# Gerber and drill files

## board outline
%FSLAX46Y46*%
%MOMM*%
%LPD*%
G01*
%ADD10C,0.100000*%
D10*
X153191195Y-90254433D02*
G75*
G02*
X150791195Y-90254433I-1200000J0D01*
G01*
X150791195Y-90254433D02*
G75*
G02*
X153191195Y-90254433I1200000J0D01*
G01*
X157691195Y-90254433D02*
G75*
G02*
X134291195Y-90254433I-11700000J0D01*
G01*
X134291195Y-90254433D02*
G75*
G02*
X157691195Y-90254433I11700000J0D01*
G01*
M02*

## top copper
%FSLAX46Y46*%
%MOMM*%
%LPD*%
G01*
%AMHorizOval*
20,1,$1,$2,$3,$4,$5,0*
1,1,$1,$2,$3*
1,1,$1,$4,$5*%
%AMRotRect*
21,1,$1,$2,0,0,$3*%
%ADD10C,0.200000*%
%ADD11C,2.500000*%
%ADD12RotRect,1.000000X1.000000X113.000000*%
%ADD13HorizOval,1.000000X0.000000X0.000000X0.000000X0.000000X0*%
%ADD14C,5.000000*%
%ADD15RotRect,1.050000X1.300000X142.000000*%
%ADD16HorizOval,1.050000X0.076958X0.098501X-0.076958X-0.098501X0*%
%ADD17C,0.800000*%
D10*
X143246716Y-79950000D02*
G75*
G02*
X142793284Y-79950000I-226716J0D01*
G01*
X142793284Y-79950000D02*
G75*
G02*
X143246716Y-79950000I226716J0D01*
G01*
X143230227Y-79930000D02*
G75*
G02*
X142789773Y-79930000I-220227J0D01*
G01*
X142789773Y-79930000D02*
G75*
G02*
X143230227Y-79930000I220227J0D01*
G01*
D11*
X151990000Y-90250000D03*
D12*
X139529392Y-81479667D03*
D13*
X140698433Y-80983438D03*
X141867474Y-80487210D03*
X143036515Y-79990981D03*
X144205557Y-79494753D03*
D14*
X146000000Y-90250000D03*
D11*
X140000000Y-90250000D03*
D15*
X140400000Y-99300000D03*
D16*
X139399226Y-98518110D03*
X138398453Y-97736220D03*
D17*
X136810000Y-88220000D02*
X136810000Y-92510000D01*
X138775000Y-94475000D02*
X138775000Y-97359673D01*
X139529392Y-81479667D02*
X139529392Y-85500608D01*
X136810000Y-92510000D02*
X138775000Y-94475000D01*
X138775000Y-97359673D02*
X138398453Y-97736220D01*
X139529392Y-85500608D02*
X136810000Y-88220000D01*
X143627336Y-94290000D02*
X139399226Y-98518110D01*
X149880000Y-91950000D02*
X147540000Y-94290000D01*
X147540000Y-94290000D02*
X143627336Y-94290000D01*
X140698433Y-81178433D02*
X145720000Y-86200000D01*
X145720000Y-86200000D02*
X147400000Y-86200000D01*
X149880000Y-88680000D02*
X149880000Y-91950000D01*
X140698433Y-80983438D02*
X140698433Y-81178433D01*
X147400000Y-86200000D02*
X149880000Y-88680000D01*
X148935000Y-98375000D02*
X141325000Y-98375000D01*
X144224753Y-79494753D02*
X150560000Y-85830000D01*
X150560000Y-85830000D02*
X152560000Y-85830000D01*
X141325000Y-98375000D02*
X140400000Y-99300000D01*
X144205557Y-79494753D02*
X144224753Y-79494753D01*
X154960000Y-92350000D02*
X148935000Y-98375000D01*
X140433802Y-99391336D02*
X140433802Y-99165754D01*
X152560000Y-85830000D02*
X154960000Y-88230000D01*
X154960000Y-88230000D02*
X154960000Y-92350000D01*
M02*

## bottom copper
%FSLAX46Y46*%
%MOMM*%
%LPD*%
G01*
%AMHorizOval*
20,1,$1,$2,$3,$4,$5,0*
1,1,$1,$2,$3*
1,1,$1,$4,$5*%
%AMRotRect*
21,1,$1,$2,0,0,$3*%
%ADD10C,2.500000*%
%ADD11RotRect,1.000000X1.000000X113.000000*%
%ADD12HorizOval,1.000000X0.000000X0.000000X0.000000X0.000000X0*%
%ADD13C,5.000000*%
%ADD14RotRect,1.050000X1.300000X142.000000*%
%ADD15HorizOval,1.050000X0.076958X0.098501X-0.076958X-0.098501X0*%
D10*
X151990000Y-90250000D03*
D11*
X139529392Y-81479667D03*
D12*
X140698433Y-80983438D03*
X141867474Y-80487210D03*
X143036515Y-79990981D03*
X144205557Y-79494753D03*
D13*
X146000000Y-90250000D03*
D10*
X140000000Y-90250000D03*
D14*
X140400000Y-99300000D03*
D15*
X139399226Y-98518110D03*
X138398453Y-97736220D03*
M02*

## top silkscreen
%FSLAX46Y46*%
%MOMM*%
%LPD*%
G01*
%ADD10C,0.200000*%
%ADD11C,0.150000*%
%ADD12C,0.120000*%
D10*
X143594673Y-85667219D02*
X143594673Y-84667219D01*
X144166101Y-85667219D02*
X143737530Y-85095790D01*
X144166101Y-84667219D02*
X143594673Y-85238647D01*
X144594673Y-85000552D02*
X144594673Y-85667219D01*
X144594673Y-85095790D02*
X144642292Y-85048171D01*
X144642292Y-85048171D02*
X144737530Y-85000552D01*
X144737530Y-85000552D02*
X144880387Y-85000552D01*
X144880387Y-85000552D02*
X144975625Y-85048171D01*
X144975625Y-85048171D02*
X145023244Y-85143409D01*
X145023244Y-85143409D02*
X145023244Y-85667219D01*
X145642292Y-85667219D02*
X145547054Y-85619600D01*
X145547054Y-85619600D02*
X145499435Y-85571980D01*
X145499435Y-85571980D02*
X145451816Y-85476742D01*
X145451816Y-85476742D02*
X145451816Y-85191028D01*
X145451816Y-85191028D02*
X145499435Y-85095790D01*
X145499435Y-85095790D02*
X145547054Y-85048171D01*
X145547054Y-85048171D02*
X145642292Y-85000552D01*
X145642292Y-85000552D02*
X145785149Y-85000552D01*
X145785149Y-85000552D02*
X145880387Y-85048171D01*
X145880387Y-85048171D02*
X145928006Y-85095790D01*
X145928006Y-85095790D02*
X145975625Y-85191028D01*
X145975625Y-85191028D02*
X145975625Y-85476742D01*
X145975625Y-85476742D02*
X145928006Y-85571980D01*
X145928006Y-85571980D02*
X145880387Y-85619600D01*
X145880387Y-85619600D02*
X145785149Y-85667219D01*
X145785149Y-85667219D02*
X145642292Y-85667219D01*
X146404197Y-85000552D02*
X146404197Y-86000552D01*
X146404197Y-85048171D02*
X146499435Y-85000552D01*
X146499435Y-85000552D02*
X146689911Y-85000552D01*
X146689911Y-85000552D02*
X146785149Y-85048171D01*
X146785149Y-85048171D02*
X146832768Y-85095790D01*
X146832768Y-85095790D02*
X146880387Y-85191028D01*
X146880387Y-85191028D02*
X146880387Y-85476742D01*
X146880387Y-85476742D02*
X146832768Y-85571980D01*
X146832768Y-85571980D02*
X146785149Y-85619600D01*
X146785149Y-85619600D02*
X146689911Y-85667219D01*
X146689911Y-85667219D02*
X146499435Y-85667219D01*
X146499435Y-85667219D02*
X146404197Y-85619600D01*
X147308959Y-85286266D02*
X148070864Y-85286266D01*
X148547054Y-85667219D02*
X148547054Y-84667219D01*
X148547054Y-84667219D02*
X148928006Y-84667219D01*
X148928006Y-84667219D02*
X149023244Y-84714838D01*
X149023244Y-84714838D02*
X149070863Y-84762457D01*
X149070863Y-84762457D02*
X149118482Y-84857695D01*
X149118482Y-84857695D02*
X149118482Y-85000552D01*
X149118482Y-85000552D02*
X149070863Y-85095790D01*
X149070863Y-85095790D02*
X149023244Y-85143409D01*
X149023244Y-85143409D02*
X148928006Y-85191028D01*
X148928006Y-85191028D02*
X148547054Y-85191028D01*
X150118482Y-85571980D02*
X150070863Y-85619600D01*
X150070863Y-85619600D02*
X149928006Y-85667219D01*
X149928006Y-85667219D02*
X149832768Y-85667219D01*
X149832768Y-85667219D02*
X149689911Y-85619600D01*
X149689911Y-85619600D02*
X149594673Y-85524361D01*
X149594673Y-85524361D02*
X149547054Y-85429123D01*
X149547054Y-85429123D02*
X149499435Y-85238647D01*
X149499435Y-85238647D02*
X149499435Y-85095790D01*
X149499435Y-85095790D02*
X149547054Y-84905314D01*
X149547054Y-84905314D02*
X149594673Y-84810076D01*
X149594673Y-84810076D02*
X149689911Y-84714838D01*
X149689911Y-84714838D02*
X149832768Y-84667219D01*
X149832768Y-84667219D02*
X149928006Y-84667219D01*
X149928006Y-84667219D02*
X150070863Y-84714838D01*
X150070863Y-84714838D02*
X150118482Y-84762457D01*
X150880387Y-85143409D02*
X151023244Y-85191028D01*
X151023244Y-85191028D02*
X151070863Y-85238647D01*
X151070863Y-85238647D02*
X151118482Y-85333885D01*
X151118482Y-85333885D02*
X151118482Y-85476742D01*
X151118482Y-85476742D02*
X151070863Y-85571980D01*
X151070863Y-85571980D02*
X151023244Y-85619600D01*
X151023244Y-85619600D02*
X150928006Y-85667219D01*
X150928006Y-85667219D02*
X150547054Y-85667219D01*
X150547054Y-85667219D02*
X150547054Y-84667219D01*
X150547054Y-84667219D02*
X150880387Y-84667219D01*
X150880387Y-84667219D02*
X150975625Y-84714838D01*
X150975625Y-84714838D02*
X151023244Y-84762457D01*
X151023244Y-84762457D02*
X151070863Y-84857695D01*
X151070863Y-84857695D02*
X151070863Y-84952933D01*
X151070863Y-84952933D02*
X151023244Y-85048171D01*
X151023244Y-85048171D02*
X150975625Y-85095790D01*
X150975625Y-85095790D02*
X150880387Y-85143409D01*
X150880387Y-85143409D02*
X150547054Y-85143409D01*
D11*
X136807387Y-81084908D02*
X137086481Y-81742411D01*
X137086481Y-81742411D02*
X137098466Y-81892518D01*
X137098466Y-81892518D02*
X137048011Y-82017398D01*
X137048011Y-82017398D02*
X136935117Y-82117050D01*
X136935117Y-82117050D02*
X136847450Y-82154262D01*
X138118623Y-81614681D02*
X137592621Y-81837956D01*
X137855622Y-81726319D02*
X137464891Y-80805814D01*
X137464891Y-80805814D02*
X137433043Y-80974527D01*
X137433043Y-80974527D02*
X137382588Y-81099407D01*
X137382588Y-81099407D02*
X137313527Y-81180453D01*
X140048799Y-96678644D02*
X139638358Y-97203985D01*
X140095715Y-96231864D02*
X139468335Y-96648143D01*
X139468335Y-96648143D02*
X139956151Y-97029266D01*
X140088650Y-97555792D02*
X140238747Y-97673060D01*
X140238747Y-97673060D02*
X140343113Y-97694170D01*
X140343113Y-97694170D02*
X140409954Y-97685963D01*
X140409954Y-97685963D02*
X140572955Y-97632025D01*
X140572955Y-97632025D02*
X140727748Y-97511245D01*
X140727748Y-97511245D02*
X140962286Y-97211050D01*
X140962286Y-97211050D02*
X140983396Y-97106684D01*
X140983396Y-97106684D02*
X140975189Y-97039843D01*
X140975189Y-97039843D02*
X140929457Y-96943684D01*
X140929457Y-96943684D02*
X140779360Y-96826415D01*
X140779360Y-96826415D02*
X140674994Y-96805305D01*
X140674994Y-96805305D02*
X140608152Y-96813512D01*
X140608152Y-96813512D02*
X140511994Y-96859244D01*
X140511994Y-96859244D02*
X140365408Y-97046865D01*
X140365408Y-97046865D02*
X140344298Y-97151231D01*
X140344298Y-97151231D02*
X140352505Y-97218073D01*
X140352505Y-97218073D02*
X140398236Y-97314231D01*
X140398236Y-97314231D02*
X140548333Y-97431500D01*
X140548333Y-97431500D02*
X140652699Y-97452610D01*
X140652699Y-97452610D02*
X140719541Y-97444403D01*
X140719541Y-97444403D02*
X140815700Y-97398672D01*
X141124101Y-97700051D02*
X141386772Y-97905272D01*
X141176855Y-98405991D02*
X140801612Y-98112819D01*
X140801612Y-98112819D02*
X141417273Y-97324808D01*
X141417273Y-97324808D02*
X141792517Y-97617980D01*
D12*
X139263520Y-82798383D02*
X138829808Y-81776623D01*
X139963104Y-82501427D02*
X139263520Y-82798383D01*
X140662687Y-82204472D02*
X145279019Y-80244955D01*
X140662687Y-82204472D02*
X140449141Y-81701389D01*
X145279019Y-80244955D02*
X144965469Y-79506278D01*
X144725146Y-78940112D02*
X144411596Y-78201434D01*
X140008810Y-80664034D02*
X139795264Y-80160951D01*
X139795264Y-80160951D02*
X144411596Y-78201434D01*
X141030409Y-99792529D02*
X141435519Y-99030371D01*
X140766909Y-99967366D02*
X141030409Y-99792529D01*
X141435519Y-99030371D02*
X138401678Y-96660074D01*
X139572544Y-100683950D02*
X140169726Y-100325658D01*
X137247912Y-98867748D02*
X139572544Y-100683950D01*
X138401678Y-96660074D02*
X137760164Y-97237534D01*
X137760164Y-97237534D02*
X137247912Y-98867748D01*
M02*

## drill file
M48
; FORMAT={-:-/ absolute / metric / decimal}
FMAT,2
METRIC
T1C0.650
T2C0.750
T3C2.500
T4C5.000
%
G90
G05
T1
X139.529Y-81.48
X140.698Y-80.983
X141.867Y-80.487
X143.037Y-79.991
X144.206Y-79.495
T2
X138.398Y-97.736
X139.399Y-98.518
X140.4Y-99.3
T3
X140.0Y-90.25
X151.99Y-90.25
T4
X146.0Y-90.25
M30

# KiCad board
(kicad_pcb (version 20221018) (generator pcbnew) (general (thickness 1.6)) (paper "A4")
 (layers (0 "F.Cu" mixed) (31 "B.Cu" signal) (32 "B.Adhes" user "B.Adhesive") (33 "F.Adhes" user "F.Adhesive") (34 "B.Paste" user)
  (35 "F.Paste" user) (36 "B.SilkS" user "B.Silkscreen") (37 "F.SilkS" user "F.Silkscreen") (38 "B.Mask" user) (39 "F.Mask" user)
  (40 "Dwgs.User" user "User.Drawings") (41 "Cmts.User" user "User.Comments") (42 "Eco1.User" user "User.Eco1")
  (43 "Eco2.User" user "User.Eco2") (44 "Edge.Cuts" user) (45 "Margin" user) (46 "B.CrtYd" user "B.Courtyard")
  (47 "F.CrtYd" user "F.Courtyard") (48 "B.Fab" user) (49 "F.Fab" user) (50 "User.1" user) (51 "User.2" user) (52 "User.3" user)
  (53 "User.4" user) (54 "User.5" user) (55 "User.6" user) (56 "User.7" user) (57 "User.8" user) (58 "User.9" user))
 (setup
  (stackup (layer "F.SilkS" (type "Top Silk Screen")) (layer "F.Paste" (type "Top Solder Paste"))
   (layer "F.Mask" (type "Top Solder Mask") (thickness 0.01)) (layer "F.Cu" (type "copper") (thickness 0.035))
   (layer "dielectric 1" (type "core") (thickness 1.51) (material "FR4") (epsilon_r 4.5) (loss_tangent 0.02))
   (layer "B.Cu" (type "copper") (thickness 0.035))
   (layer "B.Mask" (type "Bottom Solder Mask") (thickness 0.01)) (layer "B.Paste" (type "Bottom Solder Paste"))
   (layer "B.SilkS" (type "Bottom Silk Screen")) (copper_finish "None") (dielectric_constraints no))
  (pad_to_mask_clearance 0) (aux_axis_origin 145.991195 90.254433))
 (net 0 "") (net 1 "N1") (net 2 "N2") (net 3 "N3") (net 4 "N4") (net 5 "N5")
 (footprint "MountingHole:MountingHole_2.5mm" (layer "F.Cu") (at 151.99 90.25)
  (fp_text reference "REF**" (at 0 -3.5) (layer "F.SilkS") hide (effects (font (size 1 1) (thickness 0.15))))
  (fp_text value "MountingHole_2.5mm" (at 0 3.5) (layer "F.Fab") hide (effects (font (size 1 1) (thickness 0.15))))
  (pad "" thru_hole circle (at 0 0) (size 2.5 2.5) (drill 2.5) (layers "*.Cu" "*.Mask")))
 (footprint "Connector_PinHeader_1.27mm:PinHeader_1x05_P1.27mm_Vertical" (layer "F.Cu") (at 139.529392 81.479667 113)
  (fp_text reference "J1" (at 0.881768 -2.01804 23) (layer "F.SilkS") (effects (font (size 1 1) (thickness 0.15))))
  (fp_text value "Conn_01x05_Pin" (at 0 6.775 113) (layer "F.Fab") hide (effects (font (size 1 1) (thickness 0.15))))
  (fp_line (start -1.11 -0.76) (end 0 -0.76) (stroke (width 0.12) (type solid)) (layer "F.SilkS"))
  (fp_line (start -1.11 0) (end -1.11 -0.76) (stroke (width 0.12) (type solid)) (layer "F.SilkS"))
  (fp_line (start -1.11 0.76) (end -1.11 5.775) (stroke (width 0.12) (type solid)) (layer "F.SilkS"))
  (fp_line (start -1.11 0.76) (end -0.563471 0.76) (stroke (width 0.12) (type solid)) (layer "F.SilkS"))
  (fp_line (start -1.11 5.775) (end -0.30753 5.775) (stroke (width 0.12) (type solid)) (layer "F.SilkS"))
  (fp_line (start 0.30753 5.775) (end 1.11 5.775) (stroke (width 0.12) (type solid)) (layer "F.SilkS"))
  (fp_line (start 0.563471 0.76) (end 1.11 0.76) (stroke (width 0.12) (type solid)) (layer "F.SilkS"))
  (fp_line (start 1.11 0.76) (end 1.11 5.775) (stroke (width 0.12) (type solid)) (layer "F.SilkS"))
  (pad "1" thru_hole rect (at 0 0 113) (size 1 1) (drill 0.65) (layers "*.Cu" "*.Mask") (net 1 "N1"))
  (pad "2" thru_hole oval (at 0 1.27 113) (size 1 1) (drill 0.65) (layers "*.Cu" "*.Mask") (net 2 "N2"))
  (pad "3" thru_hole oval (at 0 2.54 113) (size 1 1) (drill 0.65) (layers "*.Cu" "*.Mask") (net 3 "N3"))
  (pad "4" thru_hole oval (at 0 3.81 113) (size 1 1) (drill 0.65) (layers "*.Cu" "*.Mask") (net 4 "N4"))
  (pad "5" thru_hole oval (at 0 5.08 113) (size 1 1) (drill 0.65) (layers "*.Cu" "*.Mask") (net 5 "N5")))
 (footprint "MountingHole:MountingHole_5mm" (layer "F.Cu") (at 146 90.25)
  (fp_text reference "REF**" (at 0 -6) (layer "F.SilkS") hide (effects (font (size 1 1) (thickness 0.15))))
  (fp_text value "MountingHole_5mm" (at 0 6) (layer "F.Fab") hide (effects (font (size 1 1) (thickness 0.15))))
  (pad "" thru_hole circle (at 0 0) (size 5 5) (drill 5) (layers "*.Cu" "*.Mask")))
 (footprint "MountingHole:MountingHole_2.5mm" (layer "F.Cu") (at 140 90.25)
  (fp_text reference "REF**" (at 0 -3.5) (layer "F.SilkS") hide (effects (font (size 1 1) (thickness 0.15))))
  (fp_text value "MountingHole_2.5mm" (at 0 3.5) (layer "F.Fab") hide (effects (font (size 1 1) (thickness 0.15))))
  (pad "" thru_hole circle (at 0 0) (size 2.5 2.5) (drill 2.5) (layers "*.Cu" "*.Mask")))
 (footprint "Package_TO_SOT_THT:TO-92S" (layer "F.Cu") (at 140.4 99.3 142)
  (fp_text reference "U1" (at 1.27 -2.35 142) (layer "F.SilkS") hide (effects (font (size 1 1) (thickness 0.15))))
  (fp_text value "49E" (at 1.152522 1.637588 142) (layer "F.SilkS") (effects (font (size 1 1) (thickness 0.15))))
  (fp_line (start -0.8 0) (end -0.65 0.85) (stroke (width 0.12) (type solid)) (layer "F.SilkS"))
  (fp_line (start -0.7 -0.3) (end -0.8 0) (stroke (width 0.12) (type solid)) (layer "F.SilkS"))
  (fp_line (start -0.65 0.85) (end 3.2 0.85) (stroke (width 0.12) (type solid)) (layer "F.SilkS"))
  (fp_line (start -0.2 -1.6) (end -0.45 -0.95) (stroke (width 0.12) (type solid)) (layer "F.SilkS"))
  (fp_line (start 2.75 -1.6) (end -0.2 -1.6) (stroke (width 0.12) (type solid)) (layer "F.SilkS"))
  (fp_line (start 3.2 0.85) (end 3.35 0) (stroke (width 0.12) (type solid)) (layer "F.SilkS"))
  (fp_line (start 3.35 0) (end 2.75 -1.6) (stroke (width 0.12) (type solid)) (layer "F.SilkS"))
  (pad "1" thru_hole rect (at 0 0 142) (size 1.05 1.3) (drill 0.75) (layers "*.Cu" "*.Mask") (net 5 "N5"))
  (pad "2" thru_hole oval (at 1.27 0 142) (size 1.05 1.3) (drill 0.75) (layers "*.Cu" "*.Mask") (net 2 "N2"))
  (pad "3" thru_hole oval (at 2.54 0 142) (size 1.05 1.3) (drill 0.75) (layers "*.Cu" "*.Mask") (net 1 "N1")))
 (gr_circle (center 143.02 79.95) (end 143.19 80.1) (stroke (width 0.2) (type default)) (fill none) (layer "F.Cu"))
 (gr_circle (center 143.01 79.93) (end 143.18 80.07) (stroke (width 0.2) (type default)) (fill none) (layer "F.Cu"))
 (gr_circle (center 151.991195 90.254433) (end 153.191195 90.254433) (stroke (width 0.1) (type solid)) (fill none) (layer "Edge.Cuts"))
 (gr_circle (center 145.991195 90.254433) (end 157.691195 90.254433) (stroke (width 0.1) (type default)) (fill none) (layer "Edge.Cuts"))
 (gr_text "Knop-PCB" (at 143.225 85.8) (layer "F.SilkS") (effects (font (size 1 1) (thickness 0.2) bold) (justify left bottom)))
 (segment (start 136.81 88.22) (end 136.81 92.51) (width 0.8) (layer "F.Cu") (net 1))
 (segment (start 138.775 94.475) (end 138.775 97.359673) (width 0.8) (layer "F.Cu") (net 1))
 (segment (start 139.529392 81.479667) (end 139.529392 85.500608) (width 0.8) (layer "F.Cu") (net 1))
 (segment (start 136.81 92.51) (end 138.775 94.475) (width 0.8) (layer "F.Cu") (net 1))
 (segment (start 138.775 97.359673) (end 138.398453 97.73622) (width 0.8) (layer "F.Cu") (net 1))
 (segment (start 139.529392 85.500608) (end 136.81 88.22) (width 0.8) (layer "F.Cu") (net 1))
 (segment (start 143.627336 94.29) (end 139.399226 98.51811) (width 0.8) (layer "F.Cu") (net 2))
 (segment (start 149.88 91.95) (end 147.54 94.29) (width 0.8) (layer "F.Cu") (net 2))
 (segment (start 147.54 94.29) (end 143.627336 94.29) (width 0.8) (layer "F.Cu") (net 2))
 (segment (start 140.698433 81.178433) (end 145.72 86.2) (width 0.8) (layer "F.Cu") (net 2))
 (segment (start 145.72 86.2) (end 147.4 86.2) (width 0.8) (layer "F.Cu") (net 2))
 (segment (start 149.88 88.68) (end 149.88 91.95) (width 0.8) (layer "F.Cu") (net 2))
 (segment (start 140.698433 80.983438) (end 140.698433 81.178433) (width 0.8) (layer "F.Cu") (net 2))
 (segment (start 147.4 86.2) (end 149.88 88.68) (width 0.8) (layer "F.Cu") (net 2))
 (segment (start 148.935 98.375) (end 141.325 98.375) (width 0.8) (layer "F.Cu") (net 5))
 (segment (start 144.224753 79.494753) (end 150.56 85.83) (width 0.8) (layer "F.Cu") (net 5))
 (segment (start 150.56 85.83) (end 152.56 85.83) (width 0.8) (layer "F.Cu") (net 5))
 (segment (start 141.325 98.375) (end 140.4 99.3) (width 0.8) (layer "F.Cu") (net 5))
 (segment (start 144.205557 79.494753) (end 144.224753 79.494753) (width 0.8) (layer "F.Cu") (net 5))
 (segment (start 154.96 92.35) (end 148.935 98.375) (width 0.8) (layer "F.Cu") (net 5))
 (segment (start 140.433802 99.391336) (end 140.433802 99.165754) (width 0.8) (layer "F.Cu") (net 5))
 (segment (start 152.56 85.83) (end 154.96 88.23) (width 0.8) (layer "F.Cu") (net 5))
 (segment (start 154.96 88.23) (end 154.96 92.35) (width 0.8) (layer "F.Cu") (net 5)))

